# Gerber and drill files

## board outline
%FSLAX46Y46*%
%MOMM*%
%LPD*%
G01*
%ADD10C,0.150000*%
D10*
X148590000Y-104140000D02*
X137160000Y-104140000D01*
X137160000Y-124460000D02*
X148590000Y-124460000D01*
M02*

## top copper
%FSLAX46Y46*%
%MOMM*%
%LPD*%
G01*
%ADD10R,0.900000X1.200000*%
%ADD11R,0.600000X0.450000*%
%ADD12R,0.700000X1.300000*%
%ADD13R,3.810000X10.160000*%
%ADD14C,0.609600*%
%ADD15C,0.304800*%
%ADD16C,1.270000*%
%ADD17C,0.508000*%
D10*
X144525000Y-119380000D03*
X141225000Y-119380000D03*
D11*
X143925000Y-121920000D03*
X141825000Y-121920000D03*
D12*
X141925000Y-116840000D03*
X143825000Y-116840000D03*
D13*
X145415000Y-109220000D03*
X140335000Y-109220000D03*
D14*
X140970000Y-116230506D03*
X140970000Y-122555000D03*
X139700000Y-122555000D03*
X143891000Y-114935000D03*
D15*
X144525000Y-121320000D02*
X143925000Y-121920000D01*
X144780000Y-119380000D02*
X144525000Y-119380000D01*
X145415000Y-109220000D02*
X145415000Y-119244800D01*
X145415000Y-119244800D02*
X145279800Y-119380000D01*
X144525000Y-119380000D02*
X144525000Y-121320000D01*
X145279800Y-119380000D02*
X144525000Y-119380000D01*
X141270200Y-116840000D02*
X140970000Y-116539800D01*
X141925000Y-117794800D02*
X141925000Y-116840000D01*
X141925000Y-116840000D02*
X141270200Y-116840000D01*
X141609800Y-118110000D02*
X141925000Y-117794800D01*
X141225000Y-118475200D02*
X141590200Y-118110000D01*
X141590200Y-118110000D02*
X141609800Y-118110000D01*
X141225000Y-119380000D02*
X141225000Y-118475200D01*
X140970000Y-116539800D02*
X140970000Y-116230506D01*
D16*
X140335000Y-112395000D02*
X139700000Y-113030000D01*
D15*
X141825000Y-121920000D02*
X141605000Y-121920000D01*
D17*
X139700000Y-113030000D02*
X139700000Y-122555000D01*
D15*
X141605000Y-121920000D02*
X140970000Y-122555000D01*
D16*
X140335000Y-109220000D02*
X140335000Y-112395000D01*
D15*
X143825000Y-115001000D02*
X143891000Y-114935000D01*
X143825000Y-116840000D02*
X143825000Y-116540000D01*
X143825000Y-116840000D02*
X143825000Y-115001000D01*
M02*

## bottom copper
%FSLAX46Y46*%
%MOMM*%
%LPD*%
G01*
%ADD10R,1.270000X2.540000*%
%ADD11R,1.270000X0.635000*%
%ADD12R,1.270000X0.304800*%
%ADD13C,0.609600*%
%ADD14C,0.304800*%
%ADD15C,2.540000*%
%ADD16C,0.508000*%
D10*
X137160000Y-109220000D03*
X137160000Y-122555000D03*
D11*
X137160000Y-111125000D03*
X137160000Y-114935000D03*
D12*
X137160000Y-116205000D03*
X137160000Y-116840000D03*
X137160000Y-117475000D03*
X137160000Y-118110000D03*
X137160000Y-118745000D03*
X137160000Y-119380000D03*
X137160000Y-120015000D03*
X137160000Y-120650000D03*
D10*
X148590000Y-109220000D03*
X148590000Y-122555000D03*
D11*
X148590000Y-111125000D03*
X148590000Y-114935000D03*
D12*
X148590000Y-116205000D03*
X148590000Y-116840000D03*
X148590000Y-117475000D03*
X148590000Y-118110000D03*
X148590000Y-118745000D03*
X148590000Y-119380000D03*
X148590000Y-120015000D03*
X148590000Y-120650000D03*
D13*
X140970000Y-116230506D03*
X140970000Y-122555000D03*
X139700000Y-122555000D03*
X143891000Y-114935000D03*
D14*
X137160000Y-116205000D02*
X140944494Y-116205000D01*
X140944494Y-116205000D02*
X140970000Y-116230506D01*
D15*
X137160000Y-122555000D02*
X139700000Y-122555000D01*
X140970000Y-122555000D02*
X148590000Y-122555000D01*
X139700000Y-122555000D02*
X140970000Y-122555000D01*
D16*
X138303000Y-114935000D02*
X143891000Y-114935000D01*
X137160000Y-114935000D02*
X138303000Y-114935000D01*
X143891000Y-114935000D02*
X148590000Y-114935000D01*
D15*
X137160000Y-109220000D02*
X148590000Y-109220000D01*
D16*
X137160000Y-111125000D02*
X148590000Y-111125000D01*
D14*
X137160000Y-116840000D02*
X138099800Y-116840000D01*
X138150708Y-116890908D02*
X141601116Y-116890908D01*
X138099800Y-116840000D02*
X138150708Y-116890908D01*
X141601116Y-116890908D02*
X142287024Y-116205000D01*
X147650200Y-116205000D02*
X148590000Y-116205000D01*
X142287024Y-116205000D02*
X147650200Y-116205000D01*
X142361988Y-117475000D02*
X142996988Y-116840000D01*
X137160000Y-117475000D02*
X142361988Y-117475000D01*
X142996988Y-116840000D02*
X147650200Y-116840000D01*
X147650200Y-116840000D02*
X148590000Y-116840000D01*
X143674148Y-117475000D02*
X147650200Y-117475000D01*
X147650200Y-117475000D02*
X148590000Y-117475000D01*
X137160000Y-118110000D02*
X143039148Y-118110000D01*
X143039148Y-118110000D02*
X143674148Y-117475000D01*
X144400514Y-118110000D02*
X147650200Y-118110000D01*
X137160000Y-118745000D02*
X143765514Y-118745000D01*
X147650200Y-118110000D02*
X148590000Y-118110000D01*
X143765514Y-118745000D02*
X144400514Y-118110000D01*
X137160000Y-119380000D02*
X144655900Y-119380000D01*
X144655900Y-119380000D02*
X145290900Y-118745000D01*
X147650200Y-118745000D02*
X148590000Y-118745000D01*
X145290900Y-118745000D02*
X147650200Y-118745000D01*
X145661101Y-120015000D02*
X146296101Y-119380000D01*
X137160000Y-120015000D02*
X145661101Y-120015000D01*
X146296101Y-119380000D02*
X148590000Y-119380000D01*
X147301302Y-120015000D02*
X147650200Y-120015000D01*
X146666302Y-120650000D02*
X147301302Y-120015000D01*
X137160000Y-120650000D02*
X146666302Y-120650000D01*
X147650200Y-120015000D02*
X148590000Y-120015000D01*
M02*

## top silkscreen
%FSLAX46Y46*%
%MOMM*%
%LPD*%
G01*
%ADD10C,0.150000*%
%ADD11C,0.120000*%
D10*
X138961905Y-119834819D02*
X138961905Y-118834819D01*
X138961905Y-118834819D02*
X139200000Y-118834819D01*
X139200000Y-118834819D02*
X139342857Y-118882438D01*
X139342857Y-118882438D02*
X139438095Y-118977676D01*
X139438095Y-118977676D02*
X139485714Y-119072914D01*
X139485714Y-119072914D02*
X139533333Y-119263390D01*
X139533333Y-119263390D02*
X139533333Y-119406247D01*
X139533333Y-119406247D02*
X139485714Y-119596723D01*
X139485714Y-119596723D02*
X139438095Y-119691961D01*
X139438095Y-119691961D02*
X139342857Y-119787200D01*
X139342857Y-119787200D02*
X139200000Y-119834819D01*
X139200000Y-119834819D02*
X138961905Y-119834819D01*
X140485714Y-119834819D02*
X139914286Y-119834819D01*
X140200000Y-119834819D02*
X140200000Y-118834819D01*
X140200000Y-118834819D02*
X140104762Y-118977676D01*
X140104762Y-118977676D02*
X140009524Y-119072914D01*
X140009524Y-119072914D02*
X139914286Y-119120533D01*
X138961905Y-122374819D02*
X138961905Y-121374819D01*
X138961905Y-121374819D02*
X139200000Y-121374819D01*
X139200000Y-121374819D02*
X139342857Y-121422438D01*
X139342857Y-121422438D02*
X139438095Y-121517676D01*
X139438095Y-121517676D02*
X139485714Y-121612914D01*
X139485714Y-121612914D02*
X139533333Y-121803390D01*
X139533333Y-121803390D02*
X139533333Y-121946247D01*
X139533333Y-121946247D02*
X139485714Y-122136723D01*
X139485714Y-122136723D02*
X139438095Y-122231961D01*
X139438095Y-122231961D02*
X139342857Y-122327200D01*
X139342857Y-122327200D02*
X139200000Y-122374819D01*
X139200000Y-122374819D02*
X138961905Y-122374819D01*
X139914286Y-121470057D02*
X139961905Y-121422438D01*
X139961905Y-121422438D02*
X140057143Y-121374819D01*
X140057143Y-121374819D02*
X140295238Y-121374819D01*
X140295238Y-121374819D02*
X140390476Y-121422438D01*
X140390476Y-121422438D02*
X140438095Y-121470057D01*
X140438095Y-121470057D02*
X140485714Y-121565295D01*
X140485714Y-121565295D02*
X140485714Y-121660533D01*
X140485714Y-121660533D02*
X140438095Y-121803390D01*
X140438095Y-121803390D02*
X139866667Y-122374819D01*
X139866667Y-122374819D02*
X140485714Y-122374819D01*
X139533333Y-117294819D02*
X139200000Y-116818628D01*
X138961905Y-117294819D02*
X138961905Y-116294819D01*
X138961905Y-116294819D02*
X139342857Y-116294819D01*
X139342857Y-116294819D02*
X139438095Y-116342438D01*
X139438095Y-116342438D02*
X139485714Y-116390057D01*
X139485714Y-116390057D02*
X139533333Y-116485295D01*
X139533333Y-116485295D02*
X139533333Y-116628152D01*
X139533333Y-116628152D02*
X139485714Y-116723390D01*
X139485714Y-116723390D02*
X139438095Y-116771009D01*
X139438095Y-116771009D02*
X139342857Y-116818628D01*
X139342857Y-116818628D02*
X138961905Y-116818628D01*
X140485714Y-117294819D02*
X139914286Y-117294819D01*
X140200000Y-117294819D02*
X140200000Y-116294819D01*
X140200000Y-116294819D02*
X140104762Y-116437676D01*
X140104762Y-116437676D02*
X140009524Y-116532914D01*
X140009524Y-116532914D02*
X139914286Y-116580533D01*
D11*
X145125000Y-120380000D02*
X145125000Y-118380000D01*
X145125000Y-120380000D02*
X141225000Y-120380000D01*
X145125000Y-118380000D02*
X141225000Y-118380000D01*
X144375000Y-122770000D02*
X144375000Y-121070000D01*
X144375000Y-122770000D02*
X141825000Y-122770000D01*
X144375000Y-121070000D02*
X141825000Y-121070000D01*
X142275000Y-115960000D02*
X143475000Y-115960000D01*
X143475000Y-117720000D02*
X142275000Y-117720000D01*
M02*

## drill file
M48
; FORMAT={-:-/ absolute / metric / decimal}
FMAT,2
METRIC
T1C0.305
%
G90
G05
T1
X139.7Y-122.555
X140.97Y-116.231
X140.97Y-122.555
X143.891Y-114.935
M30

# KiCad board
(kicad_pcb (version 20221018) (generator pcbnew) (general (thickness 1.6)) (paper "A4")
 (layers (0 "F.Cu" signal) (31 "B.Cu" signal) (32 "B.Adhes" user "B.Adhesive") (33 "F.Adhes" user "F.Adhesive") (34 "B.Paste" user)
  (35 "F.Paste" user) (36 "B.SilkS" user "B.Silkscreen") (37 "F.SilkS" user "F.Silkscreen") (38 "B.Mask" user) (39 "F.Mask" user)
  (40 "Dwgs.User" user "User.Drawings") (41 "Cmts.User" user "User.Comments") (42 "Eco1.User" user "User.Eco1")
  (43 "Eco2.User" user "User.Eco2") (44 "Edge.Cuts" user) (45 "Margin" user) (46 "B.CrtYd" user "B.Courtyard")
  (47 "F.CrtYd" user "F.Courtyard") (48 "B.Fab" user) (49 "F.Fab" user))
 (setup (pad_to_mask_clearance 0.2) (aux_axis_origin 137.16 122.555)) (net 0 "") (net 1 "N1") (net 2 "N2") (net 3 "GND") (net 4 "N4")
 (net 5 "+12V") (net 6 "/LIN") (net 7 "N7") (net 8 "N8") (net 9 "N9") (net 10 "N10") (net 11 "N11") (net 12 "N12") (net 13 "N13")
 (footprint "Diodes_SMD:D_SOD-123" (layer "F.Cu") (at 142.875 119.38 180)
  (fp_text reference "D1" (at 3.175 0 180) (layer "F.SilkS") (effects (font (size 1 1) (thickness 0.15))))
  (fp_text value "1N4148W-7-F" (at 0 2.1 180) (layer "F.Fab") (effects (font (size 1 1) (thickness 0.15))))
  (fp_line (start -2.25 -1) (end -2.25 1) (stroke (width 0.12) (type solid)) (layer "F.SilkS"))
  (fp_line (start -2.25 -1) (end 1.65 -1) (stroke (width 0.12) (type solid)) (layer "F.SilkS"))
  (fp_line (start -2.25 1) (end 1.65 1) (stroke (width 0.12) (type solid)) (layer "F.SilkS"))
  (pad "1" smd rect (at -1.65 0 180) (size 0.9 1.2) (layers "F.Cu" "F.Paste" "F.Mask") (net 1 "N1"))
  (pad "2" smd rect (at 1.65 0 180) (size 0.9 1.2) (layers "F.Cu" "F.Paste" "F.Mask") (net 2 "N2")))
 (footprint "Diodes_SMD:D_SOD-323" (layer "F.Cu") (at 142.875 121.92 180)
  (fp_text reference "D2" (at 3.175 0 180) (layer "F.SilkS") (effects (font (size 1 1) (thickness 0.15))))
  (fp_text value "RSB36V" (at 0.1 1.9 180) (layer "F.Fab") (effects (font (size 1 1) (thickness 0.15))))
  (fp_line (start -1.5 -0.85) (end -1.5 0.85) (stroke (width 0.12) (type solid)) (layer "F.SilkS"))
  (fp_line (start -1.5 -0.85) (end 1.05 -0.85) (stroke (width 0.12) (type solid)) (layer "F.SilkS"))
  (fp_line (start -1.5 0.85) (end 1.05 0.85) (stroke (width 0.12) (type solid)) (layer "F.SilkS"))
  (pad "1" smd rect (at -1.05 0 180) (size 0.6 0.45) (layers "F.Cu" "F.Paste" "F.Mask") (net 1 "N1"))
  (pad "2" smd rect (at 1.05 0 180) (size 0.6 0.45) (layers "F.Cu" "F.Paste" "F.Mask") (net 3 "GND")))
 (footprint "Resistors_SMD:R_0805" (layer "F.Cu") (at 142.875 116.84)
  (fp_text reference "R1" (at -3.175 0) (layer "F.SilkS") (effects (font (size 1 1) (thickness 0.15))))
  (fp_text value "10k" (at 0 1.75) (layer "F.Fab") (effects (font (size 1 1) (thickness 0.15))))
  (fp_line (start -0.6 -0.88) (end 0.6 -0.88) (stroke (width 0.12) (type solid)) (layer "F.SilkS"))
  (fp_line (start 0.6 0.88) (end -0.6 0.88) (stroke (width 0.12) (type solid)) (layer "F.SilkS"))
  (pad "1" smd rect (at -0.95 0) (size 0.7 1.3) (layers "F.Cu" "F.Paste" "F.Mask") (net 2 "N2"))
  (pad "2" smd rect (at 0.95 0) (size 0.7 1.3) (layers "F.Cu" "F.Paste" "F.Mask") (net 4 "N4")))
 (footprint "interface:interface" (layer "F.Cu") (at 137.16 104.775)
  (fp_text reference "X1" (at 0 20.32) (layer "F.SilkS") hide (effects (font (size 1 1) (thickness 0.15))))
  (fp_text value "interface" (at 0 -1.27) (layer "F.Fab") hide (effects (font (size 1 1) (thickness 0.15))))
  (pad "1" smd rect (at 0 4.445) (size 1.27 2.54) (layers "B.Cu") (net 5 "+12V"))
  (pad "2" smd rect (at 0 17.78) (size 1.27 2.54) (layers "B.Cu") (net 3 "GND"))
  (pad "3" smd rect (at 0 6.35) (size 1.27 0.635) (layers "B.Cu") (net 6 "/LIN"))
  (pad "4" smd rect (at 0 10.16) (size 1.27 0.635) (layers "B.Cu") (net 4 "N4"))
  (pad "5" smd rect (at 0 11.43) (size 1.27 0.3048) (layers "B.Cu") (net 2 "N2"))
  (pad "6" smd rect (at 0 12.065) (size 1.27 0.3048) (layers "B.Cu") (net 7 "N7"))
  (pad "7" smd rect (at 0 12.7) (size 1.27 0.3048) (layers "B.Cu") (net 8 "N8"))
  (pad "8" smd rect (at 0 13.335) (size 1.27 0.3048) (layers "B.Cu") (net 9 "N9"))
  (pad "9" smd rect (at 0 13.97) (size 1.27 0.3048) (layers "B.Cu") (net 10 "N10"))
  (pad "10" smd rect (at 0 14.605) (size 1.27 0.3048) (layers "B.Cu") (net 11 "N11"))
  (pad "11" smd rect (at 0 15.24) (size 1.27 0.3048) (layers "B.Cu") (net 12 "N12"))
  (pad "12" smd rect (at 0 15.875) (size 1.27 0.3048) (layers "B.Cu") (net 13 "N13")))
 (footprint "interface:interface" (layer "F.Cu") (at 148.59 104.775)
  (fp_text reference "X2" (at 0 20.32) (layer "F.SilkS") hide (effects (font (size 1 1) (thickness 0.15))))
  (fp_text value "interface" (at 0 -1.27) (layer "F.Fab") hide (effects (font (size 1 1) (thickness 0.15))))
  (pad "1" smd rect (at 0 4.445) (size 1.27 2.54) (layers "B.Cu") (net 5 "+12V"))
  (pad "2" smd rect (at 0 17.78) (size 1.27 2.54) (layers "B.Cu") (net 3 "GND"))
  (pad "3" smd rect (at 0 6.35) (size 1.27 0.635) (layers "B.Cu") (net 6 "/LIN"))
  (pad "4" smd rect (at 0 10.16) (size 1.27 0.635) (layers "B.Cu") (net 4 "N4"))
  (pad "5" smd rect (at 0 11.43) (size 1.27 0.3048) (layers "B.Cu") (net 7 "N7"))
  (pad "6" smd rect (at 0 12.065) (size 1.27 0.3048) (layers "B.Cu") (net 8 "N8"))
  (pad "7" smd rect (at 0 12.7) (size 1.27 0.3048) (layers "B.Cu") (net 9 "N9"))
  (pad "8" smd rect (at 0 13.335) (size 1.27 0.3048) (layers "B.Cu") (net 10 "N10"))
  (pad "9" smd rect (at 0 13.97) (size 1.27 0.3048) (layers "B.Cu") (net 11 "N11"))
  (pad "10" smd rect (at 0 14.605) (size 1.27 0.3048) (layers "B.Cu") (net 12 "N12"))
  (pad "11" smd rect (at 0 15.24) (size 1.27 0.3048) (layers "B.Cu") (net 13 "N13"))
  (pad "12" smd rect (at 0 15.875) (size 1.27 0.3048) (layers "B.Cu")))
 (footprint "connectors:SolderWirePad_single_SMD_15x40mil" (layer "F.Cu") (at 145.415 109.22)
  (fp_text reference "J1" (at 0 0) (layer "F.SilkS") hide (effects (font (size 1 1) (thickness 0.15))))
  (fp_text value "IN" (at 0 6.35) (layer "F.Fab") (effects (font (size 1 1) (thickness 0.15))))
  (pad "1" smd rect (at 0 0) (size 3.81 10.16) (layers "F.Cu" "F.Paste" "F.Mask") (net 1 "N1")))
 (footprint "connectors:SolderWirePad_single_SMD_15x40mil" (layer "F.Cu") (at 140.335 109.22)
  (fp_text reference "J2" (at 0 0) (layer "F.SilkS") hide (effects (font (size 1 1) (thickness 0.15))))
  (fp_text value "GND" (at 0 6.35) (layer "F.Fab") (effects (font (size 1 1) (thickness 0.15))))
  (pad "1" smd rect (at 0 0) (size 3.81 10.16) (layers "F.Cu" "F.Paste" "F.Mask") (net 3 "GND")))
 (gr_line (start 148.59 104.14) (end 137.16 104.14) (stroke (width 0.15) (type solid)) (layer "Edge.Cuts"))
 (gr_line (start 137.16 124.46) (end 148.59 124.46) (stroke (width 0.15) (type solid)) (layer "Edge.Cuts"))
 (segment (start 144.525 121.32) (end 143.925 121.92) (width 0.3048) (layer "F.Cu") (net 1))
 (segment (start 144.78 119.38) (end 144.525 119.38) (width 0.3048) (layer "F.Cu") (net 1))
 (segment (start 145.415 109.22) (end 145.415 119.2448) (width 0.3048) (layer "F.Cu") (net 1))
 (segment (start 145.415 119.2448) (end 145.2798 119.38) (width 0.3048) (layer "F.Cu") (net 1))
 (segment (start 144.525 119.38) (end 144.525 121.32) (width 0.3048) (layer "F.Cu") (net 1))
 (segment (start 145.2798 119.38) (end 144.525 119.38) (width 0.3048) (layer "F.Cu") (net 1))
 (segment (start 141.2702 116.84) (end 140.97 116.5398) (width 0.3048) (layer "F.Cu") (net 2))
 (segment (start 141.925 117.7948) (end 141.925 116.84) (width 0.3048) (layer "F.Cu") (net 2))
 (segment (start 141.925 116.84) (end 141.2702 116.84) (width 0.3048) (layer "F.Cu") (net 2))
 (segment (start 141.6098 118.11) (end 141.925 117.7948) (width 0.3048) (layer "F.Cu") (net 2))
 (segment (start 141.225 118.4752) (end 141.5902 118.11) (width 0.3048) (layer "F.Cu") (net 2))
 (segment (start 141.5902 118.11) (end 141.6098 118.11) (width 0.3048) (layer "F.Cu") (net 2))
 (segment (start 141.225 119.38) (end 141.225 118.4752) (width 0.3048) (layer "F.Cu") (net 2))
 (segment (start 140.97 116.5398) (end 140.97 116.230506) (width 0.3048) (layer "F.Cu") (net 2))
 (via (at 140.97 116.230506) (size 0.6096) (drill 0.3048) (layers "F.Cu" "B.Cu") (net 2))
 (segment (start 137.16 116.205) (end 140.944494 116.205) (width 0.3048) (layer "B.Cu") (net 2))
 (segment (start 140.944494 116.205) (end 140.97 116.230506) (width 0.3048) (layer "B.Cu") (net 2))
 (segment (start 140.335 112.395) (end 139.7 113.03) (width 1.27) (layer "F.Cu") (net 3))
 (segment (start 141.825 121.92) (end 141.605 121.92) (width 0.3048) (layer "F.Cu") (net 3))
 (segment (start 139.7 113.03) (end 139.7 122.555) (width 0.508) (layer "F.Cu") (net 3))
 (segment (start 141.605 121.92) (end 140.97 122.555) (width 0.3048) (layer "F.Cu") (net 3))
 (segment (start 140.335 109.22) (end 140.335 112.395) (width 1.27) (layer "F.Cu") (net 3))
 (via (at 140.97 122.555) (size 0.6096) (drill 0.3048) (layers "F.Cu" "B.Cu") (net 3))
 (via (at 139.7 122.555) (size 0.6096) (drill 0.3048) (layers "F.Cu" "B.Cu") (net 3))
 (segment (start 137.16 122.555) (end 139.7 122.555) (width 2.54) (layer "B.Cu") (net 3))
 (segment (start 140.97 122.555) (end 148.59 122.555) (width 2.54) (layer "B.Cu") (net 3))
 (segment (start 139.7 122.555) (end 140.97 122.555) (width 2.54) (layer "B.Cu") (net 3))
 (segment (start 143.825 115.001) (end 143.891 114.935) (width 0.3048) (layer "F.Cu") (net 4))
 (segment (start 143.825 116.84) (end 143.825 116.54) (width 0.3048) (layer "F.Cu") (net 4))
 (segment (start 143.825 116.84) (end 143.825 115.001) (width 0.3048) (layer "F.Cu") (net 4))
 (via (at 143.891 114.935) (size 0.6096) (drill 0.3048) (layers "F.Cu" "B.Cu") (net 4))
 (segment (start 138.303 114.935) (end 143.891 114.935) (width 0.508) (layer "B.Cu") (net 4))
 (segment (start 137.16 114.935) (end 138.303 114.935) (width 0.508) (layer "B.Cu") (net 4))
 (segment (start 143.891 114.935) (end 148.59 114.935) (width 0.508) (layer "B.Cu") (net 4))
 (segment (start 137.16 109.22) (end 148.59 109.22) (width 2.54) (layer "B.Cu") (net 5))
 (segment (start 137.16 111.125) (end 148.59 111.125) (width 0.508) (layer "B.Cu") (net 6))
 (segment (start 137.16 116.84) (end 138.0998 116.84) (width 0.3048) (layer "B.Cu") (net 7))
 (segment (start 138.150708 116.890908) (end 141.601116 116.890908) (width 0.3048) (layer "B.Cu") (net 7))
 (segment (start 138.0998 116.84) (end 138.150708 116.890908) (width 0.3048) (layer "B.Cu") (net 7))
 (segment (start 141.601116 116.890908) (end 142.287024 116.205) (width 0.3048) (layer "B.Cu") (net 7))
 (segment (start 147.6502 116.205) (end 148.59 116.205) (width 0.3048) (layer "B.Cu") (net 7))
 (segment (start 142.287024 116.205) (end 147.6502 116.205) (width 0.3048) (layer "B.Cu") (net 7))
 (segment (start 142.361988 117.475) (end 142.996988 116.84) (width 0.3048) (layer "B.Cu") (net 8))
 (segment (start 137.16 117.475) (end 142.361988 117.475) (width 0.3048) (layer "B.Cu") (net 8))
 (segment (start 142.996988 116.84) (end 147.6502 116.84) (width 0.3048) (layer "B.Cu") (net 8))
 (segment (start 147.6502 116.84) (end 148.59 116.84) (width 0.3048) (layer "B.Cu") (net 8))
 (segment (start 143.674148 117.475) (end 147.6502 117.475) (width 0.3048) (layer "B.Cu") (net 9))
 (segment (start 147.6502 117.475) (end 148.59 117.475) (width 0.3048) (layer "B.Cu") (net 9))
 (segment (start 137.16 118.11) (end 143.039148 118.11) (width 0.3048) (layer "B.Cu") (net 9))
 (segment (start 143.039148 118.11) (end 143.674148 117.475) (width 0.3048) (layer "B.Cu") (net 9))
 (segment (start 144.400514 118.11) (end 147.6502 118.11) (width 0.3048) (layer "B.Cu") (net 10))
 (segment (start 137.16 118.745) (end 143.765514 118.745) (width 0.3048) (layer "B.Cu") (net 10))
 (segment (start 147.6502 118.11) (end 148.59 118.11) (width 0.3048) (layer "B.Cu") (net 10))
 (segment (start 143.765514 118.745) (end 144.400514 118.11) (width 0.3048) (layer "B.Cu") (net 10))
 (segment (start 137.16 119.38) (end 144.6559 119.38) (width 0.3048) (layer "B.Cu") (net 11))
 (segment (start 144.6559 119.38) (end 145.2909 118.745) (width 0.3048) (layer "B.Cu") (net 11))
 (segment (start 147.6502 118.745) (end 148.59 118.745) (width 0.3048) (layer "B.Cu") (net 11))
 (segment (start 145.2909 118.745) (end 147.6502 118.745) (width 0.3048) (layer "B.Cu") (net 11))
 (segment (start 145.661101 120.015) (end 146.296101 119.38) (width 0.3048) (layer "B.Cu") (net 12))
 (segment (start 137.16 120.015) (end 145.661101 120.015) (width 0.3048) (layer "B.Cu") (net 12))
 (segment (start 146.296101 119.38) (end 148.59 119.38) (width 0.3048) (layer "B.Cu") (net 12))
 (segment (start 147.301302 120.015) (end 147.6502 120.015) (width 0.3048) (layer "B.Cu") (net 13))
 (segment (start 146.666302 120.65) (end 147.301302 120.015) (width 0.3048) (layer "B.Cu") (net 13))
 (segment (start 137.16 120.65) (end 146.666302 120.65) (width 0.3048) (layer "B.Cu") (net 13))
 (segment (start 147.6502 120.015) (end 148.59 120.015) (width 0.3048) (layer "B.Cu") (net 13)))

